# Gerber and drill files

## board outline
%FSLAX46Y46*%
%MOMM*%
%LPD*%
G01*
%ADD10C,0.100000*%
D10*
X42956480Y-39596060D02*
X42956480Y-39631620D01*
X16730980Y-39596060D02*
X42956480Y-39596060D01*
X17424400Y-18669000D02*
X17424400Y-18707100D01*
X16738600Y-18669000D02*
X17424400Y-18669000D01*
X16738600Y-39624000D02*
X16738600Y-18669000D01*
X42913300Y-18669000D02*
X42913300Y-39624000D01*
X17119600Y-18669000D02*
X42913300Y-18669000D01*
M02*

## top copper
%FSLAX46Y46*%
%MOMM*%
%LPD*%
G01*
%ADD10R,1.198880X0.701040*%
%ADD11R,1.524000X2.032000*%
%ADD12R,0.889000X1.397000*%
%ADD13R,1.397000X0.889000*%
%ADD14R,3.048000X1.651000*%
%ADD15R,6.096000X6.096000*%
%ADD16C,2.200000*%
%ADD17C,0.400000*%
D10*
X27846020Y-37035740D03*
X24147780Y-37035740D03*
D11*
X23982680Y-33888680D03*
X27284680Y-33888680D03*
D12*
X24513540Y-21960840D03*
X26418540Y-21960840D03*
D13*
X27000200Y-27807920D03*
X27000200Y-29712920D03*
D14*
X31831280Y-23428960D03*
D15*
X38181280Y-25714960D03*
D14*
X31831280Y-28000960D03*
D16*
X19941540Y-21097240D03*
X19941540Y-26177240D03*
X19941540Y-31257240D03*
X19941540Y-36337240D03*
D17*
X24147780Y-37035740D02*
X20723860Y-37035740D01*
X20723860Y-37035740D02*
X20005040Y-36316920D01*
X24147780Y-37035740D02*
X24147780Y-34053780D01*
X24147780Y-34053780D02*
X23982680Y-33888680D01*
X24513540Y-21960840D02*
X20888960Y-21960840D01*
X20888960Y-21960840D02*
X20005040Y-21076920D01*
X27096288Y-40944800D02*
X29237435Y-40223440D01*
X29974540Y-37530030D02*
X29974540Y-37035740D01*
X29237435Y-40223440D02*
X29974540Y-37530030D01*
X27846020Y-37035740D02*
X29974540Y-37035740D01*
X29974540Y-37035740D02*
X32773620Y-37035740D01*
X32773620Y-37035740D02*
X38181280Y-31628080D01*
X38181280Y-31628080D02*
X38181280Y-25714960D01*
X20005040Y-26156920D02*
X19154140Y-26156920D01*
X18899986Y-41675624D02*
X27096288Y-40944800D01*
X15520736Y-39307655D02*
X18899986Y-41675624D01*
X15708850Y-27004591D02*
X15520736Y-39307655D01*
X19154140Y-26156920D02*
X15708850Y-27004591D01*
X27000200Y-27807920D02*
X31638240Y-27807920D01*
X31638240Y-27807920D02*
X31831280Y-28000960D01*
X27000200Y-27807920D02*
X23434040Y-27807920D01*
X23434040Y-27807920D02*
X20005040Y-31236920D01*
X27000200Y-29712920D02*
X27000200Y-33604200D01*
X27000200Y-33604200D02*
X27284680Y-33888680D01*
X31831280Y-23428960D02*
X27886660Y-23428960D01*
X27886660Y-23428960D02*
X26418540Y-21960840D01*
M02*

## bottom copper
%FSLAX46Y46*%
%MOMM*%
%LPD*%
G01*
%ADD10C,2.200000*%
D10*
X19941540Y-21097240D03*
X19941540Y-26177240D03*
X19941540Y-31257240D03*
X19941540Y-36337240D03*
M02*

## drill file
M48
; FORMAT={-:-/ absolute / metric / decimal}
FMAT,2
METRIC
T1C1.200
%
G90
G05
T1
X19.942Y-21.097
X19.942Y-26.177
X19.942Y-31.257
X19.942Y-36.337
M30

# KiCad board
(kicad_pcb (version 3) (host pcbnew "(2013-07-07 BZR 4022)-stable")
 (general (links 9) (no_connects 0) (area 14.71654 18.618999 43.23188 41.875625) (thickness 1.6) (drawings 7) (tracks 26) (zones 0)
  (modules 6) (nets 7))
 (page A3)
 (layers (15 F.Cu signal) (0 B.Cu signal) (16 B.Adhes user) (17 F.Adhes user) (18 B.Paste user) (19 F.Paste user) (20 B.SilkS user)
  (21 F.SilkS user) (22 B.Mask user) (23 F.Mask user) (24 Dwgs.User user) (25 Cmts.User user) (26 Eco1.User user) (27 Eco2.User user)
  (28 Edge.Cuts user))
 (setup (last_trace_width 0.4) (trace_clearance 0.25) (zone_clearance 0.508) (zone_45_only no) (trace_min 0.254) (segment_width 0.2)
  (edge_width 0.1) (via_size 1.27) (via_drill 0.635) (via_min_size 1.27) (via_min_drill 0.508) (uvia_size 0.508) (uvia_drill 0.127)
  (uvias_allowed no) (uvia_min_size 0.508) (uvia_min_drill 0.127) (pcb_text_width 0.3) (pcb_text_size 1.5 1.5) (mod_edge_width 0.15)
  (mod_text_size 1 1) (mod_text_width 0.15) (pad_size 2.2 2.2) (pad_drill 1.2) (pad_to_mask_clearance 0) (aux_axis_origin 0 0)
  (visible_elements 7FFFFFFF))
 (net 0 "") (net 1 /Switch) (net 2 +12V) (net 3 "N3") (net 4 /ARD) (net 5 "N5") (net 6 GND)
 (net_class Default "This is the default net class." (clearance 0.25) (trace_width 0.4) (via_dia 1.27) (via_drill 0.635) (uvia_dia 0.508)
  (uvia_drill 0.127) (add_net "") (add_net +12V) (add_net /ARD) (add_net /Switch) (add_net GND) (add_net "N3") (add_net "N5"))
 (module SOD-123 (layer F.Cu) (at 25.9969 37.03574 180)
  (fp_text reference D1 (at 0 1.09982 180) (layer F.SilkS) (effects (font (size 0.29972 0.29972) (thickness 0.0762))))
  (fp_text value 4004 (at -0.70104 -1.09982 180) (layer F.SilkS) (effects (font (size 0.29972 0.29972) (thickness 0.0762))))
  (pad 1 smd rect (at -1.84912 0 180) (size 1.19888 0.70104) (layers F.Cu F.Paste F.Mask) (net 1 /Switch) (clearance 0.14986))
  (pad 2 smd rect (at 1.84912 0 180) (size 1.19888 0.70104) (layers F.Cu F.Paste F.Mask) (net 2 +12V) (clearance 0.14986)))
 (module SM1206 (layer F.Cu) (at 25.63368 33.88868)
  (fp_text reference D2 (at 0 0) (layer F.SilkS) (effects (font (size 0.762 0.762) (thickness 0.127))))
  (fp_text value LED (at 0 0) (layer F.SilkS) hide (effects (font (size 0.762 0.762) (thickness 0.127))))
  (pad 1 smd rect (at -1.651 0) (size 1.524 2.032) (layers F.Cu F.Paste F.Mask) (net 2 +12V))
  (pad 2 smd rect (at 1.651 0) (size 1.524 2.032) (layers F.Cu F.Paste F.Mask) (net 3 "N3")))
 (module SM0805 (layer F.Cu) (at 25.46604 21.96084)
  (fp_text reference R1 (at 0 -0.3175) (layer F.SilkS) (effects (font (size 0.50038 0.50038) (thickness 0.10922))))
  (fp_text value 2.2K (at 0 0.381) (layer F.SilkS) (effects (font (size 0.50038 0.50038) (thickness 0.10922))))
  (pad 1 smd rect (at -0.9525 0) (size 0.889 1.397) (layers F.Cu F.Paste F.Mask) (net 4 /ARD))
  (pad 2 smd rect (at 0.9525 0) (size 0.889 1.397) (layers F.Cu F.Paste F.Mask) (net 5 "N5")))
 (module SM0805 (layer F.Cu) (at 27.0002 28.76042 270)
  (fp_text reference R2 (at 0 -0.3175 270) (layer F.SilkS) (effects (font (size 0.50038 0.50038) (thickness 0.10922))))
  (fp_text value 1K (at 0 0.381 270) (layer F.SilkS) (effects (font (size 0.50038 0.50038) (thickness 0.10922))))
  (pad 1 smd rect (at -0.9525 0 270) (size 0.889 1.397) (layers F.Cu F.Paste F.Mask) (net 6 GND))
  (pad 2 smd rect (at 0.9525 0 270) (size 0.889 1.397) (layers F.Cu F.Paste F.Mask) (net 3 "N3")))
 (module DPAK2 (layer F.Cu) (at 31.83128 25.71496 270)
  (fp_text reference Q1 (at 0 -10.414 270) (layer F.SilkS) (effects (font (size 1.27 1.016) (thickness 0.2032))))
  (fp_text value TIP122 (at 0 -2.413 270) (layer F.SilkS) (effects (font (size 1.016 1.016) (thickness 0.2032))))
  (pad 1 smd rect (at -2.286 0 270) (size 1.651 3.048) (layers F.Cu F.Paste F.Mask) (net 5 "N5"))
  (pad 2 smd rect (at 0 -6.35 270) (size 6.096 6.096) (layers F.Cu F.Paste F.Mask) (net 1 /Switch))
  (pad 3 smd rect (at 2.286 0 270) (size 1.651 3.048) (layers F.Cu F.Paste F.Mask) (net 6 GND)))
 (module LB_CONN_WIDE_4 (layer F.Cu) (at 19.94154 26.17724 270)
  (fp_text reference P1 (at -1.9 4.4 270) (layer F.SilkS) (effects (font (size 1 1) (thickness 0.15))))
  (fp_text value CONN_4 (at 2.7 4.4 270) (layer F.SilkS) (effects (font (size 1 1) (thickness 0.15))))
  (pad 1 thru_hole circle (at -5.08 0 270) (size 2.2 2.2) (drill 1.2) (layers *.Cu *.Mask F.SilkS) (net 4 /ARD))
  (pad 2 thru_hole circle (at 0 0 270) (size 2.2 2.2) (drill 1.2) (layers *.Cu *.Mask F.SilkS) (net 1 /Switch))
  (pad 3 thru_hole circle (at 5.08 0 270) (size 2.2 2.2) (drill 1.2) (layers *.Cu *.Mask F.SilkS) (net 6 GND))
  (pad 4 thru_hole circle (at 10.16 0 270) (size 2.2 2.2) (drill 1.2) (layers *.Cu *.Mask F.SilkS) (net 2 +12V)))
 (gr_line (start 42.95648 39.59606) (end 42.95648 39.63162) (angle 90) (layer Edge.Cuts) (width 0.1))
 (gr_line (start 16.73098 39.59606) (end 42.95648 39.59606) (angle 90) (layer Edge.Cuts) (width 0.1))
 (gr_line (start 17.4244 18.669) (end 17.4244 18.7071) (angle 90) (layer Edge.Cuts) (width 0.1))
 (gr_line (start 16.7386 18.669) (end 17.4244 18.669) (angle 90) (layer Edge.Cuts) (width 0.1))
 (gr_line (start 16.7386 39.624) (end 16.7386 18.669) (angle 90) (layer Edge.Cuts) (width 0.1))
 (gr_line (start 42.9133 18.669) (end 42.9133 39.624) (angle 90) (layer Edge.Cuts) (width 0.1))
 (gr_line (start 17.1196 18.669) (end 42.9133 18.669) (angle 90) (layer Edge.Cuts) (width 0.1))
 (segment (start 24.14778 37.03574) (end 20.72386 37.03574) (width 0.4) (layer F.Cu) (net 2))
 (segment (start 20.72386 37.03574) (end 20.00504 36.31692) (width 0.4) (layer F.Cu) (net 2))
 (segment (start 24.14778 37.03574) (end 24.14778 34.05378) (width 0.4) (layer F.Cu) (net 2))
 (segment (start 24.14778 34.05378) (end 23.98268 33.88868) (width 0.4) (layer F.Cu) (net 2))
 (segment (start 24.51354 21.96084) (end 20.88896 21.96084) (width 0.4) (layer F.Cu) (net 4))
 (segment (start 20.88896 21.96084) (end 20.00504 21.07692) (width 0.4) (layer F.Cu) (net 4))
 (segment (start 27.096288 40.9448) (end 29.237435 40.22344) (width 0.4) (layer F.Cu) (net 1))
 (segment (start 29.97454 37.53003) (end 29.97454 37.03574) (width 0.4) (layer F.Cu) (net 1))
 (segment (start 29.237435 40.22344) (end 29.97454 37.53003) (width 0.4) (layer F.Cu) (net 1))
 (segment (start 27.84602 37.03574) (end 29.97454 37.03574) (width 0.4) (layer F.Cu) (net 1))
 (segment (start 29.97454 37.03574) (end 32.77362 37.03574) (width 0.4) (layer F.Cu) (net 1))
 (segment (start 32.77362 37.03574) (end 38.18128 31.62808) (width 0.4) (layer F.Cu) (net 1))
 (segment (start 38.18128 31.62808) (end 38.18128 25.71496) (width 0.4) (layer F.Cu) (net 1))
 (segment (start 20.00504 26.15692) (end 19.15414 26.15692) (width 0.4) (layer F.Cu) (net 1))
 (segment (start 18.899986 41.675624) (end 27.096288 40.9448) (width 0.4) (layer F.Cu) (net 1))
 (segment (start 15.520736 39.307655) (end 18.899986 41.675624) (width 0.4) (layer F.Cu) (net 1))
 (segment (start 15.70885 27.004591) (end 15.520736 39.307655) (width 0.4) (layer F.Cu) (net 1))
 (segment (start 19.15414 26.15692) (end 15.70885 27.004591) (width 0.4) (layer F.Cu) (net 1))
 (segment (start 27.0002 27.80792) (end 31.63824 27.80792) (width 0.4) (layer F.Cu) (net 6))
 (segment (start 31.63824 27.80792) (end 31.83128 28.00096) (width 0.4) (layer F.Cu) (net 6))
 (segment (start 27.0002 27.80792) (end 23.43404 27.80792) (width 0.4) (layer F.Cu) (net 6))
 (segment (start 23.43404 27.80792) (end 20.00504 31.23692) (width 0.4) (layer F.Cu) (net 6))
 (segment (start 27.0002 29.71292) (end 27.0002 33.6042) (width 0.4) (layer F.Cu) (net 3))
 (segment (start 27.0002 33.6042) (end 27.28468 33.88868) (width 0.4) (layer F.Cu) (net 3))
 (segment (start 31.83128 23.42896) (end 27.88666 23.42896) (width 0.4) (layer F.Cu) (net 5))
 (segment (start 27.88666 23.42896) (end 26.41854 21.96084) (width 0.4) (layer F.Cu) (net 5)))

